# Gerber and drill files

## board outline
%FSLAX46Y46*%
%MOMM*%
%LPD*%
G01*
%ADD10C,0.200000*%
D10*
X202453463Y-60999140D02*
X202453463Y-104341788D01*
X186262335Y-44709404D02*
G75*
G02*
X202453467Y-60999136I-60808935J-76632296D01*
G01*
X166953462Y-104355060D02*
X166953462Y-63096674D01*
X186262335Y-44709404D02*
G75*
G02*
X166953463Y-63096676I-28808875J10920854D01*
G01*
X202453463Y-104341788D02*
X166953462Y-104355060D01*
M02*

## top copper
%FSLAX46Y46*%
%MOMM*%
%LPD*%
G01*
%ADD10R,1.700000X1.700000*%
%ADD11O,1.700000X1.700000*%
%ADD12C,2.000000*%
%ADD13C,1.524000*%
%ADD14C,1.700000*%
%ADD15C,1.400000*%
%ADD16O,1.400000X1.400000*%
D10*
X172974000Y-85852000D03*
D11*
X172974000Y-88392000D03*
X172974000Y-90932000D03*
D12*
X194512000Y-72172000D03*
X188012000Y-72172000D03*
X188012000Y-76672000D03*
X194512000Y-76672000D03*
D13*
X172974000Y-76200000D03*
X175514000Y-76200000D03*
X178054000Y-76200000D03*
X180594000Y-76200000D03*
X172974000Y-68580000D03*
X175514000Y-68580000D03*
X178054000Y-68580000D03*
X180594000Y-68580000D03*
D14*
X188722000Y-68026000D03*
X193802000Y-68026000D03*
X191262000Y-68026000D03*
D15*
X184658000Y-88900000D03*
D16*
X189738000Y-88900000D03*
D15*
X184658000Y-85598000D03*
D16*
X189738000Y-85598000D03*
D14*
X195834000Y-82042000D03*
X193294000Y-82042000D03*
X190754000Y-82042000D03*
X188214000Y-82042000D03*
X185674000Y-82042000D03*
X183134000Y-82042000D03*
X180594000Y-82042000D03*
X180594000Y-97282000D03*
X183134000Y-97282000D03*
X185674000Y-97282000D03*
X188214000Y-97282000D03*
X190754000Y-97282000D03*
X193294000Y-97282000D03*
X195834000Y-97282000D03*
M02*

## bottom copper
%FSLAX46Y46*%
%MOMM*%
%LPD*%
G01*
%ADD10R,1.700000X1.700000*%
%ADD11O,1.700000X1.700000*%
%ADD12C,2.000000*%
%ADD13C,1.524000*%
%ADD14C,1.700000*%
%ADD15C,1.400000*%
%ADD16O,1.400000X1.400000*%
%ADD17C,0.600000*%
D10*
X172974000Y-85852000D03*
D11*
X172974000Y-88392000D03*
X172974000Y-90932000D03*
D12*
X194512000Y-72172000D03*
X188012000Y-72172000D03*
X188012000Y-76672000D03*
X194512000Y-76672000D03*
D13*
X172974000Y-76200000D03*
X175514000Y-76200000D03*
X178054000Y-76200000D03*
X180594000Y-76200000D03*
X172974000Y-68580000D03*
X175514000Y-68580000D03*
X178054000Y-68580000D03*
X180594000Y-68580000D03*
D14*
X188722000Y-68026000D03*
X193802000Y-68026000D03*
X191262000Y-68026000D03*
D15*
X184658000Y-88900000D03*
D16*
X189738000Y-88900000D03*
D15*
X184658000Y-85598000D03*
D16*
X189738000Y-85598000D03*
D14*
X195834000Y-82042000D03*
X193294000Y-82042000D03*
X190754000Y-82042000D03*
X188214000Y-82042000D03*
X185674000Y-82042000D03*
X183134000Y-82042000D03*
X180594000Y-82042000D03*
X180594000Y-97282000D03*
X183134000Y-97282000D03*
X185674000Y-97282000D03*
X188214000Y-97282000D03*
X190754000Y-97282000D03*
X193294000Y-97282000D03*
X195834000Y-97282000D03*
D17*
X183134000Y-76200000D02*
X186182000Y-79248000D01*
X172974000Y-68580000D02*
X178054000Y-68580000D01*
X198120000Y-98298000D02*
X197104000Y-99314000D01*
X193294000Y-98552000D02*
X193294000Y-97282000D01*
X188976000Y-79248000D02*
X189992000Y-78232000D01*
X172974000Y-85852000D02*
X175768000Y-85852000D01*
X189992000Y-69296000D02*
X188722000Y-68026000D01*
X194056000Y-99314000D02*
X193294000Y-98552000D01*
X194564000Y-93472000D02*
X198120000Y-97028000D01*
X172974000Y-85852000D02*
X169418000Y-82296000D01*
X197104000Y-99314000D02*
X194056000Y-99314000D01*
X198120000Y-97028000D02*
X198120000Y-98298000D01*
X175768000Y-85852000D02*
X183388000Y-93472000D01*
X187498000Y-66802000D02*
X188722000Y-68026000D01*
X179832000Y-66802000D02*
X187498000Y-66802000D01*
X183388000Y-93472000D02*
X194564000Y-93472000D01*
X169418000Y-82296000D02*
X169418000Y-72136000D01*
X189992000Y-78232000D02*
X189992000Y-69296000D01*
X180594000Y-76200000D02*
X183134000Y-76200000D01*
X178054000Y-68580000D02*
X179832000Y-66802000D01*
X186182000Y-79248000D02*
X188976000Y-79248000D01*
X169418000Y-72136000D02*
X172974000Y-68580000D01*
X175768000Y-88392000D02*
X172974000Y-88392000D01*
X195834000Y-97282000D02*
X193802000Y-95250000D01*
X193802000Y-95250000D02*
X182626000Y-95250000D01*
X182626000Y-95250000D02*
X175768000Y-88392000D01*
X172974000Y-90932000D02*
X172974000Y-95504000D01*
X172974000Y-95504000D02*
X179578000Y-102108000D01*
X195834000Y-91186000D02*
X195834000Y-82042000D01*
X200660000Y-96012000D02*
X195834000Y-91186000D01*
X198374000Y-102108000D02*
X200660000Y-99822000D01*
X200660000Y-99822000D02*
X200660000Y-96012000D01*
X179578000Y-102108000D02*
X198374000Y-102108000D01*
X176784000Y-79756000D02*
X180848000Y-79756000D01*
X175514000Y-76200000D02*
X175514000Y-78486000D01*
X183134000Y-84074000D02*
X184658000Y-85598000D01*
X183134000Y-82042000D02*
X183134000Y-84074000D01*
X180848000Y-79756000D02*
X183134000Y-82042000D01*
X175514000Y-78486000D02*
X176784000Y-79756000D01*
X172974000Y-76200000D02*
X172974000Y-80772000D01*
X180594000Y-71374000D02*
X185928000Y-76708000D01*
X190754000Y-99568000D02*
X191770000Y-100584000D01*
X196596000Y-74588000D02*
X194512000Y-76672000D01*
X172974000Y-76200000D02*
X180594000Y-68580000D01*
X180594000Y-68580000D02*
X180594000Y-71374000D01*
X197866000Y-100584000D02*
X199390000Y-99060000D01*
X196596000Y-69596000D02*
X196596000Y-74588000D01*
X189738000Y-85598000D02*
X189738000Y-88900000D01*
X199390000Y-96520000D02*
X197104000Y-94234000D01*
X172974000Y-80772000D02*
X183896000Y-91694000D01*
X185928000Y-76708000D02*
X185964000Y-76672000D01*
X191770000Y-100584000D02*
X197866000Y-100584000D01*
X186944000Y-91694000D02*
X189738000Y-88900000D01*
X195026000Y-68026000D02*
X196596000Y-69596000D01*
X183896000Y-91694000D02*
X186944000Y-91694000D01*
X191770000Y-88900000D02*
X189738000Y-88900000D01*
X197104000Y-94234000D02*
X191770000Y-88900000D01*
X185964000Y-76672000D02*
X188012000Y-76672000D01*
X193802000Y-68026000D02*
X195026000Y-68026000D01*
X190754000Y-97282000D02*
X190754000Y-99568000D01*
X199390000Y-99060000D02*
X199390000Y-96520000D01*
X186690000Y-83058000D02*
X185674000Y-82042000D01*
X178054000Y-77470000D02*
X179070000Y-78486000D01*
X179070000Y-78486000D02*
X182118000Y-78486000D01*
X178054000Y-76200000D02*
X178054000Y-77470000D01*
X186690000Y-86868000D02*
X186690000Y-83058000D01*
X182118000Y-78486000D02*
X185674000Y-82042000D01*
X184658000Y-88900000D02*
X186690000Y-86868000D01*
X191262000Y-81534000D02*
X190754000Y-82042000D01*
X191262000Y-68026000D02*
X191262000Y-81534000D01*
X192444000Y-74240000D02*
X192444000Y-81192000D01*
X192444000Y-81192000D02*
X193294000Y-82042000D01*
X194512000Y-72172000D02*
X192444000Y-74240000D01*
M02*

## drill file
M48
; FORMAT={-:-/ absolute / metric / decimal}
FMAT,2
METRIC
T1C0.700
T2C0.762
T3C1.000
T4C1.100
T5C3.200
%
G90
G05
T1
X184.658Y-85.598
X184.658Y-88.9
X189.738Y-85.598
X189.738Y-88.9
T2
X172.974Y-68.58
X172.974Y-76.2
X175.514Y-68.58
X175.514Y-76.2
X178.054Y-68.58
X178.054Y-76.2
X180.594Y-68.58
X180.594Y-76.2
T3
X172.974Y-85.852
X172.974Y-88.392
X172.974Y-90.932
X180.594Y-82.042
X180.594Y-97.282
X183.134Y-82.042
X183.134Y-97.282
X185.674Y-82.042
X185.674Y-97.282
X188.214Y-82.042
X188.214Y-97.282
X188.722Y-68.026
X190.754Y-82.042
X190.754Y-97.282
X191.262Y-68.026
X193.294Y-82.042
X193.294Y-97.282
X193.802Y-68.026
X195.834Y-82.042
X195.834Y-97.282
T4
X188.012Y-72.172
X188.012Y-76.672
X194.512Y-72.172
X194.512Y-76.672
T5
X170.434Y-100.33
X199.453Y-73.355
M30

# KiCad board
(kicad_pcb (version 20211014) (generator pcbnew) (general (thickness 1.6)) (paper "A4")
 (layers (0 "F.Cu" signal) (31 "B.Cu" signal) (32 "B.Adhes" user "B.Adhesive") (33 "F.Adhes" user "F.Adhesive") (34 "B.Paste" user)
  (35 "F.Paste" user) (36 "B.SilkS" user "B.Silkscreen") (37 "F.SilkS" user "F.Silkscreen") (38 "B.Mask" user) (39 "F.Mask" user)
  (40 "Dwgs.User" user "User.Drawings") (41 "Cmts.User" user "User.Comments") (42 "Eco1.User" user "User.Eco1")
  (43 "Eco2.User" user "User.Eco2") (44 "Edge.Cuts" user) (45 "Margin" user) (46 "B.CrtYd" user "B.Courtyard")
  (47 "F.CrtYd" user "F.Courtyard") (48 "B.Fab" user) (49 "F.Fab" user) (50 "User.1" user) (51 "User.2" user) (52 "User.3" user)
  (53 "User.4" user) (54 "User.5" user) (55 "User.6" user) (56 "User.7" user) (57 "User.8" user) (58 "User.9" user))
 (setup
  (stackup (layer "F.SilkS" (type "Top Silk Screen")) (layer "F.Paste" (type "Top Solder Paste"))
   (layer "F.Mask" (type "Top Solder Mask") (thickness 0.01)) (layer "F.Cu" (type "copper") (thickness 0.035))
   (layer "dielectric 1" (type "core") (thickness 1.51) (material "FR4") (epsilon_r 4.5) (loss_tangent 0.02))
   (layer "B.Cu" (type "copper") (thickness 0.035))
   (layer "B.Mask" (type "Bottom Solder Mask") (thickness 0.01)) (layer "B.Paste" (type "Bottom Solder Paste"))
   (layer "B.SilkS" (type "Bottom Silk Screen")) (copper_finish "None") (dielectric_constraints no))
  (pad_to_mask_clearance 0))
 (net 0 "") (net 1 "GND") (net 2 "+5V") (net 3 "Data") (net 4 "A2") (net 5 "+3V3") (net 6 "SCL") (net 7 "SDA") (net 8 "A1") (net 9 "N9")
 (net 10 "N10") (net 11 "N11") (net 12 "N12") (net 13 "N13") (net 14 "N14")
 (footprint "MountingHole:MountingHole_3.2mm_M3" (layer "F.Cu") (at 170.434 100.33)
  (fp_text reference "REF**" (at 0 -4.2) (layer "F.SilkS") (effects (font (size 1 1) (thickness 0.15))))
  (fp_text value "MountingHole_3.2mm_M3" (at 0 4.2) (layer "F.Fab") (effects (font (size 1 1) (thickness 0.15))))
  (pad "" np_thru_hole circle (at 0 0) (size 3.2 3.2) (drill 3.2) (layers *.Cu *.Mask)))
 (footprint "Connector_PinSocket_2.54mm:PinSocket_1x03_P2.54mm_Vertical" (layer "F.Cu") (at 172.974 85.852)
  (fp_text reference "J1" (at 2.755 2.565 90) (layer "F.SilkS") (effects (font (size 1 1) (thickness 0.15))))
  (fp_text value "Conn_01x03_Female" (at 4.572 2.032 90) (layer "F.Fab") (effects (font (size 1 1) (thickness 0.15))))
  (pad "1" thru_hole rect (at 0 0) (size 1.7 1.7) (drill 1) (layers *.Cu *.Mask) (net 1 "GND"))
  (pad "2" thru_hole oval (at 0 2.54) (size 1.7 1.7) (drill 1) (layers *.Cu *.Mask) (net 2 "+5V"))
  (pad "3" thru_hole oval (at 0 5.08) (size 1.7 1.7) (drill 1) (layers *.Cu *.Mask) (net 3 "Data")))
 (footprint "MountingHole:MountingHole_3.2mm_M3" (layer "F.Cu") (at 199.453462 73.35506)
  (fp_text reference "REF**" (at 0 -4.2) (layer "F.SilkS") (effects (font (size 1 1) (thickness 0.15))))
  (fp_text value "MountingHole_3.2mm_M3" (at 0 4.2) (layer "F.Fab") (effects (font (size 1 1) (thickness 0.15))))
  (pad "" np_thru_hole circle (at 0 0) (size 3.2 3.2) (drill 3.2) (layers F&B.Cu *.Mask)))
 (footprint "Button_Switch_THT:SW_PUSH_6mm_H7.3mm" (layer "F.Cu") (at 188.012 72.172)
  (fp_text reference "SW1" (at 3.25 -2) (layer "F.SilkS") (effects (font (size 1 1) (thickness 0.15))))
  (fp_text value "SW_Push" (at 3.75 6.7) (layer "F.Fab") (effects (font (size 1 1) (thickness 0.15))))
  (pad "1" thru_hole circle (at 6.5 0 90) (size 2 2) (drill 1.1) (layers *.Cu *.Mask) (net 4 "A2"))
  (pad "1" thru_hole circle (at 0 0 90) (size 2 2) (drill 1.1) (layers *.Cu *.Mask) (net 4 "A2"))
  (pad "2" thru_hole circle (at 0 4.5 90) (size 2 2) (drill 1.1) (layers *.Cu *.Mask) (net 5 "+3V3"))
  (pad "2" thru_hole circle (at 6.5 4.5 90) (size 2 2) (drill 1.1) (layers *.Cu *.Mask) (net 5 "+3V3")))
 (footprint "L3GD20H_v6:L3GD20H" (layer "F.Cu") (at 178.054 72.39 90)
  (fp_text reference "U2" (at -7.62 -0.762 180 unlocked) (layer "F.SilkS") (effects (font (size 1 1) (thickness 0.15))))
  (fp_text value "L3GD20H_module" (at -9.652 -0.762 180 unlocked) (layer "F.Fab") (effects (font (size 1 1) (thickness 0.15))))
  (pad "1" thru_hole circle (at -3.81 -5.08 90) (size 1.524 1.524) (drill 0.762) (layers *.Cu *.Mask) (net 5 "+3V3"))
  (pad "2" thru_hole circle (at -3.81 -2.54 90) (size 1.524 1.524) (drill 0.762) (layers *.Cu *.Mask) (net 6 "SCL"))
  (pad "3" thru_hole circle (at -3.81 0 90) (size 1.524 1.524) (drill 0.762) (layers *.Cu *.Mask) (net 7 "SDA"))
  (pad "4" thru_hole circle (at -3.81 2.54 90) (size 1.524 1.524) (drill 0.762) (layers *.Cu *.Mask) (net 1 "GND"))
  (pad "5" thru_hole circle (at 3.81 -5.08 90) (size 1.524 1.524) (drill 0.762) (layers *.Cu *.Mask) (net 1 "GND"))
  (pad "6" thru_hole circle (at 3.81 -2.54 90) (size 1.524 1.524) (drill 0.762) (layers *.Cu *.Mask) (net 1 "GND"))
  (pad "7" thru_hole circle (at 3.81 0 90) (size 1.524 1.524) (drill 0.762) (layers *.Cu *.Mask) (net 1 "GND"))
  (pad "8" thru_hole circle (at 3.81 2.54 90) (size 1.524 1.524) (drill 0.762) (layers *.Cu *.Mask) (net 5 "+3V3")))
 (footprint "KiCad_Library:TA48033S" (layer "F.Cu") (at 191.262 65.486)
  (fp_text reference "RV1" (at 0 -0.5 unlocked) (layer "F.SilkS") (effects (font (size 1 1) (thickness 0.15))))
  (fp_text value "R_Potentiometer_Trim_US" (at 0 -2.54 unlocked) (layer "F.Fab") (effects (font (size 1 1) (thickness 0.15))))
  (pad "1" thru_hole circle (at -2.54 2.54) (size 1.7 1.7) (drill 1) (layers *.Cu *.Mask) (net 1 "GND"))
  (pad "2" thru_hole circle (at 2.54 2.54) (size 1.7 1.7) (drill 1) (layers *.Cu *.Mask) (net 5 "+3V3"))
  (pad "3" thru_hole circle (at 0 2.54) (size 1.7 1.7) (drill 1) (layers *.Cu *.Mask) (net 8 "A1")))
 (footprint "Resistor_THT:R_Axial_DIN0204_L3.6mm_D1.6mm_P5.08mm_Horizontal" (layer "F.Cu") (at 184.658 88.9)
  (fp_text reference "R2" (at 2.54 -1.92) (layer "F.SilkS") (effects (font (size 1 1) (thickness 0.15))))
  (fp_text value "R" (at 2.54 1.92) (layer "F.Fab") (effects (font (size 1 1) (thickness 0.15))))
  (pad "1" thru_hole circle (at 0 0) (size 1.4 1.4) (drill 0.7) (layers *.Cu *.Mask) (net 7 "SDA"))
  (pad "2" thru_hole oval (at 5.08 0) (size 1.4 1.4) (drill 0.7) (layers *.Cu *.Mask) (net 5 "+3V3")))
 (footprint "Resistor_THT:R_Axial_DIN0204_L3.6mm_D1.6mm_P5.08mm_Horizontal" (layer "F.Cu") (at 184.658 85.598)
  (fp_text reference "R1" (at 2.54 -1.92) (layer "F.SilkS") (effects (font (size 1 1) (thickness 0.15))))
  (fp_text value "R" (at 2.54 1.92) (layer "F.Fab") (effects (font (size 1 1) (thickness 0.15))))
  (pad "1" thru_hole circle (at 0 0) (size 1.4 1.4) (drill 0.7) (layers *.Cu *.Mask) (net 6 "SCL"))
  (pad "2" thru_hole oval (at 5.08 0) (size 1.4 1.4) (drill 0.7) (layers *.Cu *.Mask) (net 5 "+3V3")))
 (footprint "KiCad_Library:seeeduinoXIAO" (layer "F.Cu") (at 188.214 89.662 90)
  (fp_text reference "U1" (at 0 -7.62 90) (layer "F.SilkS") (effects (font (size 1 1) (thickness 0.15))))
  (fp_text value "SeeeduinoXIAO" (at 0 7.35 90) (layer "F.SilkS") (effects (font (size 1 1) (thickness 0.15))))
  (pad "1" thru_hole circle (at 7.62 7.62 90) (size 1.7 1.7) (drill 1) (layers *.Cu *.Mask) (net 3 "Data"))
  (pad "2" thru_hole circle (at 7.62 5.08 90) (size 1.7 1.7) (drill 1) (layers *.Cu *.Mask) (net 4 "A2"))
  (pad "3" thru_hole circle (at 7.62 2.54 90) (size 1.7 1.7) (drill 1) (layers *.Cu *.Mask) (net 8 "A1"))
  (pad "4" thru_hole circle (at 7.62 0 90) (size 1.7 1.7) (drill 1) (layers *.Cu *.Mask) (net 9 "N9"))
  (pad "5" thru_hole circle (at 7.62 -2.54 90) (size 1.7 1.7) (drill 1) (layers *.Cu *.Mask) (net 7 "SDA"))
  (pad "6" thru_hole circle (at 7.62 -5.08 90) (size 1.7 1.7) (drill 1) (layers *.Cu *.Mask) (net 6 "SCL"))
  (pad "7" thru_hole circle (at 7.62 -7.62 90) (size 1.7 1.7) (drill 1) (layers *.Cu *.Mask) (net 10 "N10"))
  (pad "8" thru_hole circle (at -7.62 -7.62 90) (size 1.7 1.7) (drill 1) (layers *.Cu *.Mask) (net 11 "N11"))
  (pad "9" thru_hole circle (at -7.62 -5.08 90) (size 1.7 1.7) (drill 1) (layers *.Cu *.Mask) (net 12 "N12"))
  (pad "10" thru_hole circle (at -7.62 -2.54 90) (size 1.7 1.7) (drill 1) (layers *.Cu *.Mask) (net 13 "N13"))
  (pad "11" thru_hole circle (at -7.62 0 90) (size 1.7 1.7) (drill 1) (layers *.Cu *.Mask) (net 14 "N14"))
  (pad "12" thru_hole circle (at -7.62 2.54 90) (size 1.7 1.7) (drill 1) (layers *.Cu *.Mask) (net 5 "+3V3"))
  (pad "13" thru_hole circle (at -7.62 5.08 90) (size 1.7 1.7) (drill 1) (layers *.Cu *.Mask) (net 1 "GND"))
  (pad "14" thru_hole circle (at -7.62 7.62 90) (size 1.7 1.7) (drill 1) (layers *.Cu *.Mask) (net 2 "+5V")))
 (gr_line (start 202.453463 60.99914) (end 202.453463 104.341788) (layer "Edge.Cuts") (width 0.2))
 (gr_arc (start 186.262335 44.709404) (mid 194.837612 52.377463) (end 202.453463 60.99914) (layer "Edge.Cuts") (width 0.2))
 (gr_line (start 166.953462 104.35506) (end 166.953462 63.096674) (layer "Edge.Cuts") (width 0.2))
 (gr_arc (start 186.262335 44.709404) (mid 178.7 56.1) (end 166.953462 63.096674) (layer "Edge.Cuts") (width 0.2))
 (gr_line (start 202.453463 104.341788) (end 166.953462 104.35506) (layer "Edge.Cuts") (width 0.2))
 (segment (start 183.134 76.2) (end 186.182 79.248) (width 0.6) (layer "B.Cu") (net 1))
 (segment (start 172.974 68.58) (end 178.054 68.58) (width 0.6) (layer "B.Cu") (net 1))
 (segment (start 198.12 98.298) (end 197.104 99.314) (width 0.6) (layer "B.Cu") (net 1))
 (segment (start 193.294 98.552) (end 193.294 97.282) (width 0.6) (layer "B.Cu") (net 1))
 (segment (start 188.976 79.248) (end 189.992 78.232) (width 0.6) (layer "B.Cu") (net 1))
 (segment (start 172.974 85.852) (end 175.768 85.852) (width 0.6) (layer "B.Cu") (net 1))
 (segment (start 189.992 69.296) (end 188.722 68.026) (width 0.6) (layer "B.Cu") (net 1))
 (segment (start 194.056 99.314) (end 193.294 98.552) (width 0.6) (layer "B.Cu") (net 1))
 (segment (start 194.564 93.472) (end 198.12 97.028) (width 0.6) (layer "B.Cu") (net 1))
 (segment (start 172.974 85.852) (end 169.418 82.296) (width 0.6) (layer "B.Cu") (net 1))
 (segment (start 197.104 99.314) (end 194.056 99.314) (width 0.6) (layer "B.Cu") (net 1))
 (segment (start 198.12 97.028) (end 198.12 98.298) (width 0.6) (layer "B.Cu") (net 1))
 (segment (start 175.768 85.852) (end 183.388 93.472) (width 0.6) (layer "B.Cu") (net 1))
 (segment (start 187.498 66.802) (end 188.722 68.026) (width 0.6) (layer "B.Cu") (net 1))
 (segment (start 179.832 66.802) (end 187.498 66.802) (width 0.6) (layer "B.Cu") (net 1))
 (segment (start 183.388 93.472) (end 194.564 93.472) (width 0.6) (layer "B.Cu") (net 1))
 (segment (start 169.418 82.296) (end 169.418 72.136) (width 0.6) (layer "B.Cu") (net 1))
 (segment (start 189.992 78.232) (end 189.992 69.296) (width 0.6) (layer "B.Cu") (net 1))
 (segment (start 180.594 76.2) (end 183.134 76.2) (width 0.6) (layer "B.Cu") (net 1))
 (segment (start 178.054 68.58) (end 179.832 66.802) (width 0.6) (layer "B.Cu") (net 1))
 (segment (start 186.182 79.248) (end 188.976 79.248) (width 0.6) (layer "B.Cu") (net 1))
 (segment (start 169.418 72.136) (end 172.974 68.58) (width 0.6) (layer "B.Cu") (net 1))
 (segment (start 175.768 88.392) (end 172.974 88.392) (width 0.6) (layer "B.Cu") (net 2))
 (segment (start 195.834 97.282) (end 193.802 95.25) (width 0.6) (layer "B.Cu") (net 2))
 (segment (start 193.802 95.25) (end 182.626 95.25) (width 0.6) (layer "B.Cu") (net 2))
 (segment (start 182.626 95.25) (end 175.768 88.392) (width 0.6) (layer "B.Cu") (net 2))
 (segment (start 172.974 90.932) (end 172.974 95.504) (width 0.6) (layer "B.Cu") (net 3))
 (segment (start 172.974 95.504) (end 179.578 102.108) (width 0.6) (layer "B.Cu") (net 3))
 (segment (start 195.834 91.186) (end 195.834 82.042) (width 0.6) (layer "B.Cu") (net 3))
 (segment (start 200.66 96.012) (end 195.834 91.186) (width 0.6) (layer "B.Cu") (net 3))
 (segment (start 198.374 102.108) (end 200.66 99.822) (width 0.6) (layer "B.Cu") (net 3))
 (segment (start 200.66 99.822) (end 200.66 96.012) (width 0.6) (layer "B.Cu") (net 3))
 (segment (start 179.578 102.108) (end 198.374 102.108) (width 0.6) (layer "B.Cu") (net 3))
 (segment (start 176.784 79.756) (end 180.848 79.756) (width 0.6) (layer "B.Cu") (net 6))
 (segment (start 175.514 76.2) (end 175.514 78.486) (width 0.6) (layer "B.Cu") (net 6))
 (segment (start 183.134 84.074) (end 184.658 85.598) (width 0.6) (layer "B.Cu") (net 6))
 (segment (start 183.134 82.042) (end 183.134 84.074) (width 0.6) (layer "B.Cu") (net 6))
 (segment (start 180.848 79.756) (end 183.134 82.042) (width 0.6) (layer "B.Cu") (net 6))
 (segment (start 175.514 78.486) (end 176.784 79.756) (width 0.6) (layer "B.Cu") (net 6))
 (segment (start 172.974 76.2) (end 172.974 80.772) (width 0.6) (layer "B.Cu") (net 5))
 (segment (start 180.594 71.374) (end 185.928 76.708) (width 0.6) (layer "B.Cu") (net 5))
 (segment (start 190.754 99.568) (end 191.77 100.584) (width 0.6) (layer "B.Cu") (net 5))
 (segment (start 196.596 74.588) (end 194.512 76.672) (width 0.6) (layer "B.Cu") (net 5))
 (segment (start 172.974 76.2) (end 180.594 68.58) (width 0.6) (layer "B.Cu") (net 5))
 (segment (start 180.594 68.58) (end 180.594 71.374) (width 0.6) (layer "B.Cu") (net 5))
 (segment (start 197.866 100.584) (end 199.39 99.06) (width 0.6) (layer "B.Cu") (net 5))
 (segment (start 196.596 69.596) (end 196.596 74.588) (width 0.6) (layer "B.Cu") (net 5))
 (segment (start 189.738 85.598) (end 189.738 88.9) (width 0.6) (layer "B.Cu") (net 5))
 (segment (start 199.39 96.52) (end 197.104 94.234) (width 0.6) (layer "B.Cu") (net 5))
 (segment (start 172.974 80.772) (end 183.896 91.694) (width 0.6) (layer "B.Cu") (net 5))
 (segment (start 185.928 76.708) (end 185.964 76.672) (width 0.6) (layer "B.Cu") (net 5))
 (segment (start 191.77 100.584) (end 197.866 100.584) (width 0.6) (layer "B.Cu") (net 5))
 (segment (start 186.944 91.694) (end 189.738 88.9) (width 0.6) (layer "B.Cu") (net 5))
 (segment (start 195.026 68.026) (end 196.596 69.596) (width 0.6) (layer "B.Cu") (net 5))
 (segment (start 183.896 91.694) (end 186.944 91.694) (width 0.6) (layer "B.Cu") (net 5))
 (segment (start 191.77 88.9) (end 189.738 88.9) (width 0.6) (layer "B.Cu") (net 5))
 (segment (start 197.104 94.234) (end 191.77 88.9) (width 0.6) (layer "B.Cu") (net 5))
 (segment (start 185.964 76.672) (end 188.012 76.672) (width 0.6) (layer "B.Cu") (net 5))
 (segment (start 193.802 68.026) (end 195.026 68.026) (width 0.6) (layer "B.Cu") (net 5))
 (segment (start 190.754 97.282) (end 190.754 99.568) (width 0.6) (layer "B.Cu") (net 5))
 (segment (start 199.39 99.06) (end 199.39 96.52) (width 0.6) (layer "B.Cu") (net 5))
 (segment (start 186.69 83.058) (end 185.674 82.042) (width 0.6) (layer "B.Cu") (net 7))
 (segment (start 178.054 77.47) (end 179.07 78.486) (width 0.6) (layer "B.Cu") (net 7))
 (segment (start 179.07 78.486) (end 182.118 78.486) (width 0.6) (layer "B.Cu") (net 7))
 (segment (start 178.054 76.2) (end 178.054 77.47) (width 0.6) (layer "B.Cu") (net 7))
 (segment (start 186.69 86.868) (end 186.69 83.058) (width 0.6) (layer "B.Cu") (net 7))
 (segment (start 182.118 78.486) (end 185.674 82.042) (width 0.6) (layer "B.Cu") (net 7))
 (segment (start 184.658 88.9) (end 186.69 86.868) (width 0.6) (layer "B.Cu") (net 7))
 (segment (start 191.262 81.534) (end 190.754 82.042) (width 0.6) (layer "B.Cu") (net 8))
 (segment (start 191.262 68.026) (end 191.262 81.534) (width 0.6) (layer "B.Cu") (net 8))
 (segment (start 192.444 74.24) (end 192.444 81.192) (width 0.6) (layer "B.Cu") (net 4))
 (segment (start 192.444 81.192) (end 193.294 82.042) (width 0.6) (layer "B.Cu") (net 4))
 (segment (start 194.512 72.172) (end 192.444 74.24) (width 0.6) (layer "B.Cu") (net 4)))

